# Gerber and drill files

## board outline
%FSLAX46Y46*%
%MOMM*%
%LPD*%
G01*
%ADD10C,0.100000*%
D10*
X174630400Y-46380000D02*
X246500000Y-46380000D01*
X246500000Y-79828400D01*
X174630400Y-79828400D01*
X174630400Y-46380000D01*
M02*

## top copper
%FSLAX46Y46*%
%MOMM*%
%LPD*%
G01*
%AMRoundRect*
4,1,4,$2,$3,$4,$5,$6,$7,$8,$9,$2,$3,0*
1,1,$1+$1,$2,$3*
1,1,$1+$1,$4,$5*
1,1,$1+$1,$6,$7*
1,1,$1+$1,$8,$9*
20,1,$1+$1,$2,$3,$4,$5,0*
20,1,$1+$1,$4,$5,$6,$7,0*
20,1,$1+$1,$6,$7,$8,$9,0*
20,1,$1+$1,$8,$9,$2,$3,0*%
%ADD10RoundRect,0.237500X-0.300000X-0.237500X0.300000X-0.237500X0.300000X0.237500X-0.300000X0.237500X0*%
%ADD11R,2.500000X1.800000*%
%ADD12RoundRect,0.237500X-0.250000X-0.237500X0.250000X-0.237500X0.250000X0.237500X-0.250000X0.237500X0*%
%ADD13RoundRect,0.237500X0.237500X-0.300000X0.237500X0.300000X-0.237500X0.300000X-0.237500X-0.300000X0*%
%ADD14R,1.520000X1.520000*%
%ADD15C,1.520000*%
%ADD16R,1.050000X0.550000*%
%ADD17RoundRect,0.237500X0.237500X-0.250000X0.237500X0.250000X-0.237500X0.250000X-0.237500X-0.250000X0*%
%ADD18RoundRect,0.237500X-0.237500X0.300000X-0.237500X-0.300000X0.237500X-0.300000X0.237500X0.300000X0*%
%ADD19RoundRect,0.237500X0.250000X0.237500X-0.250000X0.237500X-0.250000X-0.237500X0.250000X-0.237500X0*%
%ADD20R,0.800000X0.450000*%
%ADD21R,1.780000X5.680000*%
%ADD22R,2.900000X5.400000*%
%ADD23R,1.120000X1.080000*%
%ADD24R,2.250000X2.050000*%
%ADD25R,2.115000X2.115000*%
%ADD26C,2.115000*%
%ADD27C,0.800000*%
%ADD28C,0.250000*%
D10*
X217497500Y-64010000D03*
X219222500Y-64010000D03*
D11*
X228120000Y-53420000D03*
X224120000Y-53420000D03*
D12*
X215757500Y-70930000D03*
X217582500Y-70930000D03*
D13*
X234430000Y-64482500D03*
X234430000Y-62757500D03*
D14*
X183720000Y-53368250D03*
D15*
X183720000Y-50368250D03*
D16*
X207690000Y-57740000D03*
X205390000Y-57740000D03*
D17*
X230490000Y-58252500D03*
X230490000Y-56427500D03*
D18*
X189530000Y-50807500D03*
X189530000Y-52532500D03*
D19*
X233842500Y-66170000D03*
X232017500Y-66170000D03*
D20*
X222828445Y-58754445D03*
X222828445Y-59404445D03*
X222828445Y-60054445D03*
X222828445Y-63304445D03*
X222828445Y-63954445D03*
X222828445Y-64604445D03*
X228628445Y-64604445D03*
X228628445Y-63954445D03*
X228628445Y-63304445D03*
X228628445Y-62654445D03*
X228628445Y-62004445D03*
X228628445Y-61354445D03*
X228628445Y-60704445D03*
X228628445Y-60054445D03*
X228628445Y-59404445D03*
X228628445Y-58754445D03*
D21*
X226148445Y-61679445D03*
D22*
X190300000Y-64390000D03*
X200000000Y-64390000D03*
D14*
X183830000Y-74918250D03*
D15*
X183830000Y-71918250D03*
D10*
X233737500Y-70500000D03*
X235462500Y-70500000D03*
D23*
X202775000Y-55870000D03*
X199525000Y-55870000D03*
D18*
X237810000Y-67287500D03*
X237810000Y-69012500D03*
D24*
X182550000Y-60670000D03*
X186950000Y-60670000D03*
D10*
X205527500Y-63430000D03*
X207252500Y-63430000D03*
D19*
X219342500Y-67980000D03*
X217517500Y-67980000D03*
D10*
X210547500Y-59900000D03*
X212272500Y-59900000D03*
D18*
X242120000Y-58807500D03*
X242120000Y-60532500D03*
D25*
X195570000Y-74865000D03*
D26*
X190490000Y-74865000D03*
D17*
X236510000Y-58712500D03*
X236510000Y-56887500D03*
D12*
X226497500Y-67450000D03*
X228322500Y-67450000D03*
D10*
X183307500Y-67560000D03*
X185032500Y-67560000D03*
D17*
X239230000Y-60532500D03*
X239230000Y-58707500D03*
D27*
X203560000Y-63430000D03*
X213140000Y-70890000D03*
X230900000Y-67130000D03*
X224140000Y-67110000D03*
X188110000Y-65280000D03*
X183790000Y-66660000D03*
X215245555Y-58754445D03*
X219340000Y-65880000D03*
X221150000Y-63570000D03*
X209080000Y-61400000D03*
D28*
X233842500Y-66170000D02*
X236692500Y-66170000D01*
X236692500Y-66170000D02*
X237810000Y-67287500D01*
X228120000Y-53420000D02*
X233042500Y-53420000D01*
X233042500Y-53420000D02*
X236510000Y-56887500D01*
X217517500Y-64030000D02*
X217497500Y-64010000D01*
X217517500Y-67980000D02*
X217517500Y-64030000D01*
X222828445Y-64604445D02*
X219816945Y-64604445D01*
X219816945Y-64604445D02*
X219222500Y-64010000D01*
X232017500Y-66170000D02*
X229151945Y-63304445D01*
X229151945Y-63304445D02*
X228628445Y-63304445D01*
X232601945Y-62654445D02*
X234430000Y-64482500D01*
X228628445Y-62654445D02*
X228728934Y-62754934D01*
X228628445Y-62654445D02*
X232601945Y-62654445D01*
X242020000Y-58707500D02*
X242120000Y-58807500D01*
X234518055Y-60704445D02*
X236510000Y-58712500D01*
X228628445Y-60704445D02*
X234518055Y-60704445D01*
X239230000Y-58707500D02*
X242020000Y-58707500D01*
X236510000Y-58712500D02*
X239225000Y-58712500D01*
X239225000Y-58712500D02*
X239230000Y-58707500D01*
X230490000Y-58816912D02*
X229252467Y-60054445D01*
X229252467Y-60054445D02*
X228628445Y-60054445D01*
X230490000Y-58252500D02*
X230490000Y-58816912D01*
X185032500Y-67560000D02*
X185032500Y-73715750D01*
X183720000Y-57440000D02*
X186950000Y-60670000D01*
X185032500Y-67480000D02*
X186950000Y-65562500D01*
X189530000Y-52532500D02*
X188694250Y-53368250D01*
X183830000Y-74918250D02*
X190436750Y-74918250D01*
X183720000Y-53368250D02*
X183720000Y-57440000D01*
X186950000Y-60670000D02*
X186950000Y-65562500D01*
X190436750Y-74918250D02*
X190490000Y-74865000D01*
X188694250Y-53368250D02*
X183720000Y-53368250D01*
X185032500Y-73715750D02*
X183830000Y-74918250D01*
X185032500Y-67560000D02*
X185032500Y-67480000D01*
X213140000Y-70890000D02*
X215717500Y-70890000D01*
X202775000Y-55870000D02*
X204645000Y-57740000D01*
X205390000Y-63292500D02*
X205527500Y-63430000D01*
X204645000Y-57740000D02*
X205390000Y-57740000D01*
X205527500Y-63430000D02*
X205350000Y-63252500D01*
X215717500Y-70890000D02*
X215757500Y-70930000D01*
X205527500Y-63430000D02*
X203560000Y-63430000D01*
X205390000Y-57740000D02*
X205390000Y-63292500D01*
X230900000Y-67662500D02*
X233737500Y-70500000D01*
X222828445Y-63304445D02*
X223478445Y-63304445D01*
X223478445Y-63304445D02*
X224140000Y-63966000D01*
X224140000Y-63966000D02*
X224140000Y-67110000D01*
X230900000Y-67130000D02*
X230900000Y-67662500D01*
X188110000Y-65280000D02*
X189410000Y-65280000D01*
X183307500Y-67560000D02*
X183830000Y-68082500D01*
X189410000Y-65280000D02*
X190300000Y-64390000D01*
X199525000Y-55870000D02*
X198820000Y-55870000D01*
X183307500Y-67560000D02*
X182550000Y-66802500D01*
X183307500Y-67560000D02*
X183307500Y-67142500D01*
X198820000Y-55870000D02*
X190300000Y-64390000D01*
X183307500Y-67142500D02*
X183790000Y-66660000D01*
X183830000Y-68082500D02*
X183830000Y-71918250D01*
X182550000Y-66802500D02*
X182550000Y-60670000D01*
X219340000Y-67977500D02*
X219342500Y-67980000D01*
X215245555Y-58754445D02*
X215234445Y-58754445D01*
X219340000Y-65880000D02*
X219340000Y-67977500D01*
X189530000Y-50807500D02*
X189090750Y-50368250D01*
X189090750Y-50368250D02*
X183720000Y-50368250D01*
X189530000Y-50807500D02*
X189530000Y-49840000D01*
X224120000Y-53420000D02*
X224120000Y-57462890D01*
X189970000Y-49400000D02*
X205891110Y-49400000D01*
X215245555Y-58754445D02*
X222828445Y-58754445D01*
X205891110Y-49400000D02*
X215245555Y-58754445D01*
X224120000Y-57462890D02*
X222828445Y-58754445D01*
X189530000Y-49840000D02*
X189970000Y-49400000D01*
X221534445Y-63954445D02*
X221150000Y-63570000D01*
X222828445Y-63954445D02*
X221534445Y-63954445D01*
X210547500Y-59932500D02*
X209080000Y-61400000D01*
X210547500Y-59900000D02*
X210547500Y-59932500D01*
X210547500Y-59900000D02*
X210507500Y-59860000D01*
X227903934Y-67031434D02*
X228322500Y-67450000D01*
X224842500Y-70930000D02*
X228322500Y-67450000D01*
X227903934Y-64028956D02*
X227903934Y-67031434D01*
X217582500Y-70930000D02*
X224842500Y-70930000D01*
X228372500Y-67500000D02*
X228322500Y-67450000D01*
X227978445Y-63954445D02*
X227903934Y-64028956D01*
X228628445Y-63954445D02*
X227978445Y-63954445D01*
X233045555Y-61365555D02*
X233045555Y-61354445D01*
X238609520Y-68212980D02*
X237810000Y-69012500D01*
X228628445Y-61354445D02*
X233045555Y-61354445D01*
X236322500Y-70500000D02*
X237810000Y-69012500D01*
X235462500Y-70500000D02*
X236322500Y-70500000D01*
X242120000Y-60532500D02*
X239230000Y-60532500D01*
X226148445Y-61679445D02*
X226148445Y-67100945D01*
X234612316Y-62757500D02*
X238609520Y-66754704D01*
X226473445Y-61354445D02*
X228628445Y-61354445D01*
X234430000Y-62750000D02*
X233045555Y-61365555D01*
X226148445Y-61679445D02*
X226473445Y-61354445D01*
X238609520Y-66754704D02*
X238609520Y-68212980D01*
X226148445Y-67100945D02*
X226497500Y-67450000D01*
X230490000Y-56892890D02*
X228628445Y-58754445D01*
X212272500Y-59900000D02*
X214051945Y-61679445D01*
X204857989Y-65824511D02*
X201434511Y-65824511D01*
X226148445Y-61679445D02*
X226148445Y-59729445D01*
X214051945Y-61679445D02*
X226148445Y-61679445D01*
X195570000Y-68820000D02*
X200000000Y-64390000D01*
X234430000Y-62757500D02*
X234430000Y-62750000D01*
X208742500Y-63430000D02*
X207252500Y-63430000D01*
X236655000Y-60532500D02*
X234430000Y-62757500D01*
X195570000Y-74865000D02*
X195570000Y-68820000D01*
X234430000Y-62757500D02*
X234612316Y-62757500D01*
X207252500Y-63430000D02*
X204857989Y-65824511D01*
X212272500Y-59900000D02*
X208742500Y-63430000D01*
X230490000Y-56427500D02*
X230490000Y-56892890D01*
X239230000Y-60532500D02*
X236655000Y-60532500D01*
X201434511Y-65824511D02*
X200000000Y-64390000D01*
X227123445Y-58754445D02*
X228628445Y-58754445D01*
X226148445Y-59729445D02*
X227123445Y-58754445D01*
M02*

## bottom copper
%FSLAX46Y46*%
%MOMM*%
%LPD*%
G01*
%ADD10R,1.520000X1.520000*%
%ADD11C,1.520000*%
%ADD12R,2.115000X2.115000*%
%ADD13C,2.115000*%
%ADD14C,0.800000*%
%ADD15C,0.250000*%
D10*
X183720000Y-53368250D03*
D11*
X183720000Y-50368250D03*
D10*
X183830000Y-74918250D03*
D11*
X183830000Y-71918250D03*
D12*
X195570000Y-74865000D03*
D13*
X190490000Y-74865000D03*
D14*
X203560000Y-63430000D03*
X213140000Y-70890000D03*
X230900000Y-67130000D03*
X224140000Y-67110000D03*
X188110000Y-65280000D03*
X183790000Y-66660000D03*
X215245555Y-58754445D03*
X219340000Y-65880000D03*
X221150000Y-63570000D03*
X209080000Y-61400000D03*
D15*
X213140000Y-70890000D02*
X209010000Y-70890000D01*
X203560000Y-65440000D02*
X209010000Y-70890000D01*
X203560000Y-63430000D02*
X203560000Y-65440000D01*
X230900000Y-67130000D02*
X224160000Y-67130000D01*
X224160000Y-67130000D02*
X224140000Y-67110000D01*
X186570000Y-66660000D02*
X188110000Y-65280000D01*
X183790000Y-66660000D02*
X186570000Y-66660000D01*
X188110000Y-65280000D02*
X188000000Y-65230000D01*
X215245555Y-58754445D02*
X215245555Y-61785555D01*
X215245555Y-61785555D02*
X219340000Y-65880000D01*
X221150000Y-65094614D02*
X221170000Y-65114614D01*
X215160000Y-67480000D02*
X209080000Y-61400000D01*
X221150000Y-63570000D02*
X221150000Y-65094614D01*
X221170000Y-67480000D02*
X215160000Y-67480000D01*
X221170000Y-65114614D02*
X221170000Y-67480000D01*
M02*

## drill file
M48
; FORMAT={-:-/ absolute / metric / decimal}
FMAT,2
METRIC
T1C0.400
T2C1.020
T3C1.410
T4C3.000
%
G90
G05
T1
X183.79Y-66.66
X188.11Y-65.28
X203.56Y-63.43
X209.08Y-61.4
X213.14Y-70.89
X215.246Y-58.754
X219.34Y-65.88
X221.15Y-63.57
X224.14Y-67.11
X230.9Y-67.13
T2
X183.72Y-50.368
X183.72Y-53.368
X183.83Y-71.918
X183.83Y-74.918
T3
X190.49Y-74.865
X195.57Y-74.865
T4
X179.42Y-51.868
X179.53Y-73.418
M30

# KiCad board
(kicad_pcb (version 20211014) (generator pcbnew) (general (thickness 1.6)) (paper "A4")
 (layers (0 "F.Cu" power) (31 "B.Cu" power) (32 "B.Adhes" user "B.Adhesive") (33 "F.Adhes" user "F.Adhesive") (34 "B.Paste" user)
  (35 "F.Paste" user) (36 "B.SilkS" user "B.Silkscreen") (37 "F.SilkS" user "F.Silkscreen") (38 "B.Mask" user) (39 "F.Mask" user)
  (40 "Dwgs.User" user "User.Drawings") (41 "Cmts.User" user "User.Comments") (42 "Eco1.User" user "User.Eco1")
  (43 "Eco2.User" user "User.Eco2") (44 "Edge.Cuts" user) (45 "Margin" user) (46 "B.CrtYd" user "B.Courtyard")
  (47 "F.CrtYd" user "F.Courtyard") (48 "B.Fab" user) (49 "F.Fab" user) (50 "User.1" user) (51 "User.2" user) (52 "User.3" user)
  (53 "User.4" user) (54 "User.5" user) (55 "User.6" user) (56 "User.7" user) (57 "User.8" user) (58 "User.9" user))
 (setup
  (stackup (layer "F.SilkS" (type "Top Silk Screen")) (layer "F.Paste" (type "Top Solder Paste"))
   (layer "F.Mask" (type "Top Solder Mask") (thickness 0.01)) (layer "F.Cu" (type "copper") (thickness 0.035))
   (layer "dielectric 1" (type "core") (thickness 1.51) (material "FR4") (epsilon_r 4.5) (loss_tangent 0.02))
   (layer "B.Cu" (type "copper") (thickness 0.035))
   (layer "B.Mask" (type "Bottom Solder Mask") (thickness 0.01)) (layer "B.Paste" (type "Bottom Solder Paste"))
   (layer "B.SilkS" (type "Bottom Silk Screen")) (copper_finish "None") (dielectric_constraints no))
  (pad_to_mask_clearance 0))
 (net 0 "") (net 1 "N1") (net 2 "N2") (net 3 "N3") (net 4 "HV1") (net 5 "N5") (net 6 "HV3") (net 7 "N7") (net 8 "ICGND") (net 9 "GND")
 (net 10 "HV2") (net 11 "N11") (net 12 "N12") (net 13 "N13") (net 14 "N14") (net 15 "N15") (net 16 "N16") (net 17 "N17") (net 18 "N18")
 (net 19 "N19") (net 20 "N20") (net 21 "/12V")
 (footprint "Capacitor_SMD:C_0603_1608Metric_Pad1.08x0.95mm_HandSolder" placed (layer "F.Cu") (at 218.36 64.01)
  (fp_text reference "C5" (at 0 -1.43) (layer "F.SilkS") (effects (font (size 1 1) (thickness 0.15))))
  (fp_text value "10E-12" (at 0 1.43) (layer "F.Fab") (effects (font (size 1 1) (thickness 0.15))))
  (pad "1" smd roundrect locked (at -0.8625 0) (size 1.075 0.95) (layers "F.Cu" "F.Paste" "F.Mask") (roundrect_rratio 0.25) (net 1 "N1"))
  (pad "2" smd roundrect locked (at 0.8625 0) (size 1.075 0.95) (layers "F.Cu" "F.Paste" "F.Mask") (roundrect_rratio 0.25) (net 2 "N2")))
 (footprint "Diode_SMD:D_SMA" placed (layer "F.Cu") (at 226.12 53.42 180)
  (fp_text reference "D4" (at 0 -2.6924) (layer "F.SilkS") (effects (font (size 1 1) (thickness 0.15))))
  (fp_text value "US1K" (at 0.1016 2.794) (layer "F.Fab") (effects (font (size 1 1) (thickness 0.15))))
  (pad "1" smd rect locked (at -2 0 180) (size 2.5 1.8) (layers "F.Cu" "F.Paste" "F.Mask") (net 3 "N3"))
  (pad "2" smd rect locked (at 2 0 180) (size 2.5 1.8) (layers "F.Cu" "F.Paste" "F.Mask") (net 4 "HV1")))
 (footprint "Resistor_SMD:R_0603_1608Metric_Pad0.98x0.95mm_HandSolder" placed (layer "F.Cu") (at 216.67 70.93)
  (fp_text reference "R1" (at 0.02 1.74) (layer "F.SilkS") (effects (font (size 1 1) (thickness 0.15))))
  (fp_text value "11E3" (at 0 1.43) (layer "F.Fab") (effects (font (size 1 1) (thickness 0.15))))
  (pad "1" smd roundrect locked (at -0.9125 0) (size 0.975 0.95) (layers "F.Cu" "F.Paste" "F.Mask") (roundrect_rratio 0.25) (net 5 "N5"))
  (pad "2" smd roundrect locked (at 0.9125 0) (size 0.975 0.95) (layers "F.Cu" "F.Paste" "F.Mask") (roundrect_rratio 0.25) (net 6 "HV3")))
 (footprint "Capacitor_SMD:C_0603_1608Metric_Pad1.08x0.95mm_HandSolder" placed (layer "F.Cu") (at 234.43 63.62 90)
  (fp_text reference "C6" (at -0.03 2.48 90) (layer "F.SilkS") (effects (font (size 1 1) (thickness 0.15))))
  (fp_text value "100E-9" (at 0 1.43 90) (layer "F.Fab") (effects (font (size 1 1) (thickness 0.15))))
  (pad "1" smd roundrect locked (at -0.8625 0 90) (size 1.075 0.95) (layers "F.Cu" "F.Paste" "F.Mask") (roundrect_rratio 0.25) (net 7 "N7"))
  (pad "2" smd roundrect locked (at 0.8625 0 90) (size 1.075 0.95) (layers "F.Cu" "F.Paste" "F.Mask") (roundrect_rratio 0.25)
   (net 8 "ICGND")))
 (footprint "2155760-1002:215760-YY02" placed (layer "F.Cu") (at 183.72 53.36825 -90)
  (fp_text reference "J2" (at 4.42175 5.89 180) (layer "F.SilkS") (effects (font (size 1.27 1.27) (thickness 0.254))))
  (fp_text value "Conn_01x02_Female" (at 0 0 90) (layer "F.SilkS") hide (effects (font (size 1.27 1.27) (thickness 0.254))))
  (pad "" np_thru_hole circle locked (at -1.5 4.3 270) (size 3 3) (drill 3) (layers *.Cu *.Mask))
  (pad "1" thru_hole rect locked (at 0 0 270) (size 1.52 1.52) (drill 1.02) (layers *.Cu *.Mask) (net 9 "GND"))
  (pad "2" thru_hole circle locked (at -3 0 270) (size 1.52 1.52) (drill 1.02) (layers *.Cu *.Mask) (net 4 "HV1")))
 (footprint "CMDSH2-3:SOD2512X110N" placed (layer "F.Cu") (at 206.54 57.74 180)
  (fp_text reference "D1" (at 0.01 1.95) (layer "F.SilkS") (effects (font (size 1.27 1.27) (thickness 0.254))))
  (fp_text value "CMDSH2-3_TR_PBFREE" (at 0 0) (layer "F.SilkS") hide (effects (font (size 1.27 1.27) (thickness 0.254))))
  (pad "1" smd rect locked (at -1.15 0 270) (size 0.55 1.05) (layers "F.Cu" "F.Paste" "F.Mask") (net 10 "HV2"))
  (pad "2" smd rect locked (at 1.15 0 270) (size 0.55 1.05) (layers "F.Cu" "F.Paste" "F.Mask") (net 5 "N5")))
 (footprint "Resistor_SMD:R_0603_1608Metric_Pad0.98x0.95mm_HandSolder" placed (layer "F.Cu") (at 230.49 57.34 90)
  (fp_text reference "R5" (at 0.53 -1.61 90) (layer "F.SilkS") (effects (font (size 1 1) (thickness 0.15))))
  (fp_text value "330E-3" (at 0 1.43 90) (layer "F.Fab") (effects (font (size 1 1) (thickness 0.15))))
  (pad "1" smd roundrect locked (at -0.9125 0 90) (size 0.975 0.95) (layers "F.Cu" "F.Paste" "F.Mask") (roundrect_rratio 0.25)
   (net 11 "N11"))
  (pad "2" smd roundrect locked (at 0.9125 0 90) (size 0.975 0.95) (layers "F.Cu" "F.Paste" "F.Mask") (roundrect_rratio 0.25)
   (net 8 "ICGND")))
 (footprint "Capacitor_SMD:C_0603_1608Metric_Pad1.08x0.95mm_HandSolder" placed (layer "F.Cu") (at 189.53 51.67 -90)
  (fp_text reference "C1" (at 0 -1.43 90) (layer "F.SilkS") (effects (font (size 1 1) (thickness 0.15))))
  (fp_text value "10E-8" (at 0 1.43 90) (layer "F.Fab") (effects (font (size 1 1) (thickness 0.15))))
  (pad "1" smd roundrect locked (at -0.8625 0 270) (size 1.075 0.95) (layers "F.Cu" "F.Paste" "F.Mask") (roundrect_rratio 0.25)
   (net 4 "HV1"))
  (pad "2" smd roundrect locked (at 0.8625 0 270) (size 1.075 0.95) (layers "F.Cu" "F.Paste" "F.Mask") (roundrect_rratio 0.25) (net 9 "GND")))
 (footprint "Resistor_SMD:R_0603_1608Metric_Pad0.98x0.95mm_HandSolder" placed (layer "F.Cu") (at 232.93 66.17 180)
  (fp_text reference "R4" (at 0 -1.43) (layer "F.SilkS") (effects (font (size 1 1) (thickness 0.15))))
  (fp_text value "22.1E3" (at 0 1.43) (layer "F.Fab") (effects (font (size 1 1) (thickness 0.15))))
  (pad "1" smd roundrect locked (at -0.9125 0 180) (size 0.975 0.95) (layers "F.Cu" "F.Paste" "F.Mask") (roundrect_rratio 0.25)
   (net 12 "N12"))
  (pad "2" smd roundrect locked (at 0.9125 0 180) (size 0.975 0.95) (layers "F.Cu" "F.Paste" "F.Mask") (roundrect_rratio 0.25)
   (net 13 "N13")))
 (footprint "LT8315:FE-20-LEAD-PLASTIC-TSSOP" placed (layer "F.Cu") (at 225.728445 61.679445 -90)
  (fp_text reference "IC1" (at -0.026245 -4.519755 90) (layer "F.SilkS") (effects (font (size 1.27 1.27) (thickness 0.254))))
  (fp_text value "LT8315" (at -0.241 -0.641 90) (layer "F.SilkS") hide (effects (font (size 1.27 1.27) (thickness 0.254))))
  (pad "1" smd rect (at -2.925 2.9 270) (size 0.45 0.8) (layers "F.Cu" "F.Paste" "F.Mask") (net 4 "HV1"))
  (pad "2" smd rect (at -2.275 2.9 270) (size 0.45 0.8) (layers "F.Cu" "F.Paste" "F.Mask") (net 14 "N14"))
  (pad "3" smd rect (at -1.625 2.9 270) (size 0.45 0.8) (layers "F.Cu" "F.Paste" "F.Mask") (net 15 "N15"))
  (pad "8" smd rect (at 1.625 2.9 270) (size 0.45 0.8) (layers "F.Cu" "F.Paste" "F.Mask") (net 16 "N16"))
  (pad "9" smd rect (at 2.275 2.9 270) (size 0.45 0.8) (layers "F.Cu" "F.Paste" "F.Mask") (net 10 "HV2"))
  (pad "10" smd rect (at 2.925 2.9 270) (size 0.45 0.8) (layers "F.Cu" "F.Paste" "F.Mask") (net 2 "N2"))
  (pad "11" smd rect (at 2.925 -2.9 270) (size 0.45 0.8) (layers "F.Cu" "F.Paste" "F.Mask") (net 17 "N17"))
  (pad "12" smd rect (at 2.275 -2.9 270) (size 0.45 0.8) (layers "F.Cu" "F.Paste" "F.Mask") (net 6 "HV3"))
  (pad "13" smd rect (at 1.625 -2.9 270) (size 0.45 0.8) (layers "F.Cu" "F.Paste" "F.Mask") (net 13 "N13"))
  (pad "14" smd rect (at 0.975 -2.9 270) (size 0.45 0.8) (layers "F.Cu" "F.Paste" "F.Mask") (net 7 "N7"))
  (pad "15" smd rect (at 0.325 -2.9 270) (size 0.45 0.8) (layers "F.Cu" "F.Paste" "F.Mask") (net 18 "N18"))
  (pad "16" smd rect (at -0.325 -2.9 270) (size 0.45 0.8) (layers "F.Cu" "F.Paste" "F.Mask") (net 8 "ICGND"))
  (pad "17" smd rect (at -0.975 -2.9 270) (size 0.45 0.8) (layers "F.Cu" "F.Paste" "F.Mask") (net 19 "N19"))
  (pad "18" smd rect (at -1.625 -2.9 270) (size 0.45 0.8) (layers "F.Cu" "F.Paste" "F.Mask") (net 11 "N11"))
  (pad "19" smd rect (at -2.275 -2.9 270) (size 0.45 0.8) (layers "F.Cu" "F.Paste" "F.Mask") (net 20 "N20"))
  (pad "20" smd rect (at -2.925 -2.9 270) (size 0.45 0.8) (layers "F.Cu" "F.Paste" "F.Mask") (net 8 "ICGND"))
  (pad "21" smd rect (at 0 -0.42) (size 1.78 5.68) (layers "F.Cu" "F.Paste" "F.Mask") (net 8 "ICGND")))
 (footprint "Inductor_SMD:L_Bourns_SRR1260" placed (layer "F.Cu") (at 195.15 64.39)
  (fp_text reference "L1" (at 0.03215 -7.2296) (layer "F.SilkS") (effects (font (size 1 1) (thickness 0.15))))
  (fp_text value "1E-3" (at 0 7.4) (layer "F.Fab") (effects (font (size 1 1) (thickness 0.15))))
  (pad "1" smd rect locked (at -4.85 0) (size 2.9 5.4) (layers "F.Cu" "F.Paste" "F.Mask") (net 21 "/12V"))
  (pad "2" smd rect locked (at 4.85 0) (size 2.9 5.4) (layers "F.Cu" "F.Paste" "F.Mask") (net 8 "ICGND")))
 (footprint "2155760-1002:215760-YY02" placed (layer "F.Cu") (at 183.83 74.91825 -90)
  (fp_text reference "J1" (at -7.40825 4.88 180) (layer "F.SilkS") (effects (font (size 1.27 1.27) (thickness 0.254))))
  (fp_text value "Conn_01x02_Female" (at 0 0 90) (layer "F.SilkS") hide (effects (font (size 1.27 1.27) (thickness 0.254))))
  (pad "" np_thru_hole circle locked (at -1.5 4.3 270) (size 3 3) (drill 3) (layers *.Cu *.Mask))
  (pad "1" thru_hole rect locked (at 0 0 270) (size 1.52 1.52) (drill 1.02) (layers *.Cu *.Mask) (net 9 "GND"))
  (pad "2" thru_hole circle locked (at -3 0 270) (size 1.52 1.52) (drill 1.02) (layers *.Cu *.Mask) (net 21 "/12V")))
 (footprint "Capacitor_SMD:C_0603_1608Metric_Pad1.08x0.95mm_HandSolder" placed (layer "F.Cu") (at 234.6 70.5)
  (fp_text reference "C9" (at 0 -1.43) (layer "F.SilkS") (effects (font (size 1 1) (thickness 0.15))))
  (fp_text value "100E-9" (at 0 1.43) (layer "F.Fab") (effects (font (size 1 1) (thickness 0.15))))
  (pad "1" smd roundrect locked (at -0.8625 0) (size 1.075 0.95) (layers "F.Cu" "F.Paste" "F.Mask") (roundrect_rratio 0.25) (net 16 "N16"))
  (pad "2" smd roundrect locked (at 0.8625 0) (size 1.075 0.95) (layers "F.Cu" "F.Paste" "F.Mask") (roundrect_rratio 0.25) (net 8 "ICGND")))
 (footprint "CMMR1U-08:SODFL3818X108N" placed (layer "F.Cu") (at 201.15 55.87 180)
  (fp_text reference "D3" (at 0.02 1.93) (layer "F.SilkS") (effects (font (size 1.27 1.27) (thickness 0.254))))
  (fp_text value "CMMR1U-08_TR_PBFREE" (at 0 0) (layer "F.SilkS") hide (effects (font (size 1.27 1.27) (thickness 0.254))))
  (pad "1" smd rect locked (at -1.625 0 270) (size 1.08 1.12) (layers "F.Cu" "F.Paste" "F.Mask") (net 5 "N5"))
  (pad "2" smd rect locked (at 1.625 0 270) (size 1.08 1.12) (layers "F.Cu" "F.Paste" "F.Mask") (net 21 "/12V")))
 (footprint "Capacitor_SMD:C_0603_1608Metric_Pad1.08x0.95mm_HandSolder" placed (layer "F.Cu") (at 237.81 68.15 -90)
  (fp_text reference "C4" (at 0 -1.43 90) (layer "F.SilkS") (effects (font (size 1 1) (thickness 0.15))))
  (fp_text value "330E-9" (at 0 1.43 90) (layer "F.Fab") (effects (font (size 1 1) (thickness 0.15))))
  (pad "1" smd roundrect locked (at -0.8625 0 270) (size 1.075 0.95) (layers "F.Cu" "F.Paste" "F.Mask") (roundrect_rratio 0.25)
   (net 12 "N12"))
  (pad "2" smd roundrect locked (at 0.8625 0 270) (size 1.075 0.95) (layers "F.Cu" "F.Paste" "F.Mask") (roundrect_rratio 0.25)
   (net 8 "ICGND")))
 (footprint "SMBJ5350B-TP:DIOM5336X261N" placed (layer "F.Cu") (at 184.75 60.67)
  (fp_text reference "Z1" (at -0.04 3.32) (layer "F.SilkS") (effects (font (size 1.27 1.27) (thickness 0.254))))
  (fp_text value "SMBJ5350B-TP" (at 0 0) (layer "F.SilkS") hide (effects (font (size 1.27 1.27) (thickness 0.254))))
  (pad "1" smd rect (at -2.2 0 90) (size 2.05 2.25) (layers "F.Cu" "F.Paste" "F.Mask") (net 21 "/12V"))
  (pad "2" smd rect (at 2.2 0 90) (size 2.05 2.25) (layers "F.Cu" "F.Paste" "F.Mask") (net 9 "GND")))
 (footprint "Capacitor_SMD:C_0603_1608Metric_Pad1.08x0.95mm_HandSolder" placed (layer "F.Cu") (at 206.39 63.43)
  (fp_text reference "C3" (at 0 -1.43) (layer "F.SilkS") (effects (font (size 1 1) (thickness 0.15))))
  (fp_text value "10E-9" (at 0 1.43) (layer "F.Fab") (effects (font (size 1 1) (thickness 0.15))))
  (pad "1" smd roundrect locked (at -0.8625 0) (size 1.075 0.95) (layers "F.Cu" "F.Paste" "F.Mask") (roundrect_rratio 0.25) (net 5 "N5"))
  (pad "2" smd roundrect locked (at 0.8625 0) (size 1.075 0.95) (layers "F.Cu" "F.Paste" "F.Mask") (roundrect_rratio 0.25) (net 8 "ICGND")))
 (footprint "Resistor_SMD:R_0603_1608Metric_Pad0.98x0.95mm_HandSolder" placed (layer "F.Cu") (at 218.43 67.98 180)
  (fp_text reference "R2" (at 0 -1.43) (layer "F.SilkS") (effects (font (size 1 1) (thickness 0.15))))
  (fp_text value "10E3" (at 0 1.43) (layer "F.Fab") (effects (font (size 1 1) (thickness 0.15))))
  (pad "1" smd roundrect locked (at -0.9125 0 180) (size 0.975 0.95) (layers "F.Cu" "F.Paste" "F.Mask") (roundrect_rratio 0.25)
   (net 4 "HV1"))
  (pad "2" smd roundrect locked (at 0.9125 0 180) (size 0.975 0.95) (layers "F.Cu" "F.Paste" "F.Mask") (roundrect_rratio 0.25) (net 1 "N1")))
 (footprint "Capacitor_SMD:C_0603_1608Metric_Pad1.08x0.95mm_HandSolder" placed (layer "F.Cu") (at 211.41 59.9)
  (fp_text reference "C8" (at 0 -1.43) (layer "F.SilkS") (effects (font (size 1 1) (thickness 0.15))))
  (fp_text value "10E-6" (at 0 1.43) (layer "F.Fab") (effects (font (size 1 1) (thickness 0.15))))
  (pad "1" smd roundrect locked (at -0.8625 0) (size 1.075 0.95) (layers "F.Cu" "F.Paste" "F.Mask") (roundrect_rratio 0.25) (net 10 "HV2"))
  (pad "2" smd roundrect locked (at 0.8625 0) (size 1.075 0.95) (layers "F.Cu" "F.Paste" "F.Mask") (roundrect_rratio 0.25) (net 8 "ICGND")))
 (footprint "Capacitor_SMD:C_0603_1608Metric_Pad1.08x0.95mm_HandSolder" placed (layer "F.Cu") (at 242.12 59.67 -90)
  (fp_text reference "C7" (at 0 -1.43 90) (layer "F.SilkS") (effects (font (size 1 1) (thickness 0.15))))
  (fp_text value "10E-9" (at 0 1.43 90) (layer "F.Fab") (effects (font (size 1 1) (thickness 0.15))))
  (pad "1" smd roundrect locked (at -0.8625 0 270) (size 1.075 0.95) (layers "F.Cu" "F.Paste" "F.Mask") (roundrect_rratio 0.25)
   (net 19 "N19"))
  (pad "2" smd roundrect locked (at 0.8625 0 270) (size 1.075 0.95) (layers "F.Cu" "F.Paste" "F.Mask") (roundrect_rratio 0.25)
   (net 8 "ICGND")))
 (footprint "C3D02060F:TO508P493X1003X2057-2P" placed (layer "F.Cu") (at 195.57 74.865 180)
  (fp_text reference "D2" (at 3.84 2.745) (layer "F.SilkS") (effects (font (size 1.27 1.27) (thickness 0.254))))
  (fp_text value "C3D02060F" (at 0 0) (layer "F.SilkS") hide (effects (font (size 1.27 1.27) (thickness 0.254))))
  (pad "1" thru_hole rect (at 0 0 180) (size 2.115 2.115) (drill 1.41) (layers *.Cu *.Mask) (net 8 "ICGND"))
  (pad "2" thru_hole circle (at 5.08 0 180) (size 2.115 2.115) (drill 1.41) (layers *.Cu *.Mask) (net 9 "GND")))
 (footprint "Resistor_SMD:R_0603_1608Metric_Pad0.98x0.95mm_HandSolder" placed (layer "F.Cu") (at 236.51 57.8 90)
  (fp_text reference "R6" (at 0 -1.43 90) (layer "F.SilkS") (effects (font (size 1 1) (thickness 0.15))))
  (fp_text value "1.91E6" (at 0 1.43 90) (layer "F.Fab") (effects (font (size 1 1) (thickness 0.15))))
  (pad "1" smd roundrect locked (at -0.9125 0 90) (size 0.975 0.95) (layers "F.Cu" "F.Paste" "F.Mask") (roundrect_rratio 0.25)
   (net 19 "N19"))
  (pad "2" smd roundrect locked (at 0.9125 0 90) (size 0.975 0.95) (layers "F.Cu" "F.Paste" "F.Mask") (roundrect_rratio 0.25) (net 3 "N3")))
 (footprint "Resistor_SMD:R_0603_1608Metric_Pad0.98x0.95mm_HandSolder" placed (layer "F.Cu") (at 227.41 67.45)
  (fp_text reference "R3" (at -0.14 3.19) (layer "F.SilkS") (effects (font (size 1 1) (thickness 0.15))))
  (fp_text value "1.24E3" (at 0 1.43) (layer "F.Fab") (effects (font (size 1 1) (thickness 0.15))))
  (pad "1" smd roundrect locked (at -0.9125 0) (size 0.975 0.95) (layers "F.Cu" "F.Paste" "F.Mask") (roundrect_rratio 0.25) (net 8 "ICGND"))
  (pad "2" smd roundrect locked (at 0.9125 0) (size 0.975 0.95) (layers "F.Cu" "F.Paste" "F.Mask") (roundrect_rratio 0.25) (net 6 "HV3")))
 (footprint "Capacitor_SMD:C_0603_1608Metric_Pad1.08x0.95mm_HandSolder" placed (layer "F.Cu") (at 184.17 67.56)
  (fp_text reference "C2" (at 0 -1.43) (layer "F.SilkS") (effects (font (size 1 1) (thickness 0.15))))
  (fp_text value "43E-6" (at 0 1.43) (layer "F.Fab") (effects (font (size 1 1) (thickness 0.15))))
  (pad "1" smd roundrect locked (at -0.8625 0) (size 1.075 0.95) (layers "F.Cu" "F.Paste" "F.Mask") (roundrect_rratio 0.25) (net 21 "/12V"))
  (pad "2" smd roundrect locked (at 0.8625 0) (size 1.075 0.95) (layers "F.Cu" "F.Paste" "F.Mask") (roundrect_rratio 0.25) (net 9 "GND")))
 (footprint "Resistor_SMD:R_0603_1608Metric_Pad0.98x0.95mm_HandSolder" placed (layer "F.Cu") (at 239.23 59.62 90)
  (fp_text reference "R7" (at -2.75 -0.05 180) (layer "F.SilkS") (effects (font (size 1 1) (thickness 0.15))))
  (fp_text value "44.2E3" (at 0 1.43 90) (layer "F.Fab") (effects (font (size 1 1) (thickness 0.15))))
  (pad "1" smd roundrect locked (at -0.9125 0 90) (size 0.975 0.95) (layers "F.Cu" "F.Paste" "F.Mask") (roundrect_rratio 0.25)
   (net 8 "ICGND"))
  (pad "2" smd roundrect locked (at 0.9125 0 90) (size 0.975 0.95) (layers "F.Cu" "F.Paste" "F.Mask") (roundrect_rratio 0.25) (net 19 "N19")))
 (gr_rect (start 174.6304 46.38) (end 246.5 79.8284) (layer "Edge.Cuts") (width 0.1) (fill none))
 (segment (start 233.8425 66.17) (end 236.6925 66.17) (width 0.25) (layer "F.Cu") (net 12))
 (segment (start 236.6925 66.17) (end 237.81 67.2875) (width 0.25) (layer "F.Cu") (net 12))
 (segment (start 228.12 53.42) (end 233.0425 53.42) (width 0.25) (layer "F.Cu") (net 3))
 (segment (start 233.0425 53.42) (end 236.51 56.8875) (width 0.25) (layer "F.Cu") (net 3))
 (segment (start 217.5175 64.03) (end 217.4975 64.01) (width 0.25) (layer "F.Cu") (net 1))
 (segment (start 217.5175 67.98) (end 217.5175 64.03) (width 0.25) (layer "F.Cu") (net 1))
 (segment (start 222.828445 64.604445) (end 219.816945 64.604445) (width 0.25) (layer "F.Cu") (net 2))
 (segment (start 219.816945 64.604445) (end 219.2225 64.01) (width 0.25) (layer "F.Cu") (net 2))
 (segment (start 232.0175 66.17) (end 229.151945 63.304445) (width 0.25) (layer "F.Cu") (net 13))
 (segment (start 229.151945 63.304445) (end 228.628445 63.304445) (width 0.25) (layer "F.Cu") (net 13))
 (segment (start 232.601945 62.654445) (end 234.43 64.4825) (width 0.25) (layer "F.Cu") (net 7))
 (segment (start 228.628445 62.654445) (end 228.728934 62.754934) (width 0.25) (layer "F.Cu") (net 7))
 (segment (start 228.628445 62.654445) (end 232.601945 62.654445) (width 0.25) (layer "F.Cu") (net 7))
 (segment (start 242.02 58.7075) (end 242.12 58.8075) (width 0.25) (layer "F.Cu") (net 19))
 (segment (start 234.518055 60.704445) (end 236.51 58.7125) (width 0.25) (layer "F.Cu") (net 19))
 (segment (start 228.628445 60.704445) (end 234.518055 60.704445) (width 0.25) (layer "F.Cu") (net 19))
 (segment (start 239.23 58.7075) (end 242.02 58.7075) (width 0.25) (layer "F.Cu") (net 19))
 (segment (start 236.51 58.7125) (end 239.225 58.7125) (width 0.25) (layer "F.Cu") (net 19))
 (segment (start 239.225 58.7125) (end 239.23 58.7075) (width 0.25) (layer "F.Cu") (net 19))
 (segment (start 230.49 58.816912) (end 229.252467 60.054445) (width 0.25) (layer "F.Cu") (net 11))
 (segment (start 229.252467 60.054445) (end 228.628445 60.054445) (width 0.25) (layer "F.Cu") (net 11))
 (segment (start 230.49 58.2525) (end 230.49 58.816912) (width 0.25) (layer "F.Cu") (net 11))
 (segment (start 185.0325 67.56) (end 185.0325 73.71575) (width 0.25) (layer "F.Cu") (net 9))
 (segment (start 183.72 57.44) (end 186.95 60.67) (width 0.25) (layer "F.Cu") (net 9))
 (segment (start 185.0325 67.48) (end 186.95 65.5625) (width 0.25) (layer "F.Cu") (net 9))
 (segment (start 189.53 52.5325) (end 188.69425 53.36825) (width 0.25) (layer "F.Cu") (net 9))
 (segment (start 183.83 74.91825) (end 190.43675 74.91825) (width 0.25) (layer "F.Cu") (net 9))
 (segment (start 183.72 53.36825) (end 183.72 57.44) (width 0.25) (layer "F.Cu") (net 9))
 (segment (start 186.95 60.67) (end 186.95 65.5625) (width 0.25) (layer "F.Cu") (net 9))
 (segment (start 190.43675 74.91825) (end 190.49 74.865) (width 0.25) (layer "F.Cu") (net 9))
 (segment (start 188.69425 53.36825) (end 183.72 53.36825) (width 0.25) (layer "F.Cu") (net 9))
 (segment (start 185.0325 73.71575) (end 183.83 74.91825) (width 0.25) (layer "F.Cu") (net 9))
 (segment (start 185.0325 67.56) (end 185.0325 67.48) (width 0.25) (layer "F.Cu") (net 9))
 (segment (start 213.14 70.89) (end 215.7175 70.89) (width 0.25) (layer "F.Cu") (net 5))
 (segment (start 202.775 55.87) (end 204.645 57.74) (width 0.25) (layer "F.Cu") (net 5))
 (segment (start 205.39 63.2925) (end 205.5275 63.43) (width 0.25) (layer "F.Cu") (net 5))
 (segment (start 204.645 57.74) (end 205.39 57.74) (width 0.25) (layer "F.Cu") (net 5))
 (segment (start 205.5275 63.43) (end 205.35 63.2525) (width 0.25) (layer "F.Cu") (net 5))
 (segment (start 215.7175 70.89) (end 215.7575 70.93) (width 0.25) (layer "F.Cu") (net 5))
 (segment (start 205.5275 63.43) (end 203.56 63.43) (width 0.25) (layer "F.Cu") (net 5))
 (segment (start 205.39 57.74) (end 205.39 63.2925) (width 0.25) (layer "F.Cu") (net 5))
 (via (at 203.56 63.43) (size 0.8) (drill 0.4) (layers "F.Cu" "B.Cu") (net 5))
 (via (at 213.14 70.89) (size 0.8) (drill 0.4) (layers "F.Cu" "B.Cu") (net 5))
 (segment (start 213.14 70.89) (end 209.01 70.89) (width 0.25) (layer "B.Cu") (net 5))
 (segment (start 203.56 65.44) (end 209.01 70.89) (width 0.25) (layer "B.Cu") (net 5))
 (segment (start 203.56 63.43) (end 203.56 65.44) (width 0.25) (layer "B.Cu") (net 5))
 (segment (start 230.9 67.6625) (end 233.7375 70.5) (width 0.25) (layer "F.Cu") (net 16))
 (segment (start 222.828445 63.304445) (end 223.478445 63.304445) (width 0.25) (layer "F.Cu") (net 16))
 (segment (start 223.478445 63.304445) (end 224.14 63.966) (width 0.25) (layer "F.Cu") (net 16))
 (segment (start 224.14 63.966) (end 224.14 67.11) (width 0.25) (layer "F.Cu") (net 16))
 (segment (start 230.9 67.13) (end 230.9 67.6625) (width 0.25) (layer "F.Cu") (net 16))
 (via (at 230.9 67.13) (size 0.8) (drill 0.4) (layers "F.Cu" "B.Cu") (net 16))
 (via (at 224.14 67.11) (size 0.8) (drill 0.4) (layers "F.Cu" "B.Cu") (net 16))
 (segment (start 230.9 67.13) (end 224.16 67.13) (width 0.25) (layer "B.Cu") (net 16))
 (segment (start 224.16 67.13) (end 224.14 67.11) (width 0.25) (layer "B.Cu") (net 16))
 (segment (start 188.11 65.28) (end 189.41 65.28) (width 0.25) (layer "F.Cu") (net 21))
 (segment (start 183.3075 67.56) (end 183.83 68.0825) (width 0.25) (layer "F.Cu") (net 21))
 (segment (start 189.41 65.28) (end 190.3 64.39) (width 0.25) (layer "F.Cu") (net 21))
 (segment (start 199.525 55.87) (end 198.82 55.87) (width 0.25) (layer "F.Cu") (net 21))
 (segment (start 183.3075 67.56) (end 182.55 66.8025) (width 0.25) (layer "F.Cu") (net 21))
 (segment (start 183.3075 67.56) (end 183.3075 67.1425) (width 0.25) (layer "F.Cu") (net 21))
 (segment (start 198.82 55.87) (end 190.3 64.39) (width 0.25) (layer "F.Cu") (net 21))
 (segment (start 183.3075 67.1425) (end 183.79 66.66) (width 0.25) (layer "F.Cu") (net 21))
 (segment (start 183.83 68.0825) (end 183.83 71.91825) (width 0.25) (layer "F.Cu") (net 21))
 (segment (start 182.55 66.8025) (end 182.55 60.67) (width 0.25) (layer "F.Cu") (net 21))
 (via (at 188.11 65.28) (size 0.8) (drill 0.4) (layers "F.Cu" "B.Cu") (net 21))
 (via (at 183.79 66.66) (size 0.8) (drill 0.4) (layers "F.Cu" "B.Cu") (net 21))
 (segment (start 186.57 66.66) (end 188.11 65.28) (width 0.25) (layer "B.Cu") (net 21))
 (segment (start 183.79 66.66) (end 186.57 66.66) (width 0.25) (layer "B.Cu") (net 21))
 (segment (start 188.11 65.28) (end 188 65.23) (width 0.25) (layer "B.Cu") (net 21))
 (segment (start 219.34 67.9775) (end 219.3425 67.98) (width 0.25) (layer "F.Cu") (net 4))
 (segment (start 215.245555 58.754445) (end 215.234445 58.754445) (width 0.25) (layer "F.Cu") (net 4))
 (segment (start 219.34 65.88) (end 219.34 67.9775) (width 0.25) (layer "F.Cu") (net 4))
 (segment (start 189.53 50.8075) (end 189.09075 50.36825) (width 0.25) (layer "F.Cu") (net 4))
 (segment (start 189.09075 50.36825) (end 183.72 50.36825) (width 0.25) (layer "F.Cu") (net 4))
 (segment (start 189.53 50.8075) (end 189.53 49.84) (width 0.25) (layer "F.Cu") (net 4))
 (segment (start 224.12 53.42) (end 224.12 57.46289) (width 0.25) (layer "F.Cu") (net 4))
 (segment (start 189.97 49.4) (end 205.89111 49.4) (width 0.25) (layer "F.Cu") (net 4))
 (segment (start 215.245555 58.754445) (end 222.828445 58.754445) (width 0.25) (layer "F.Cu") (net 4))
 (segment (start 205.89111 49.4) (end 215.245555 58.754445) (width 0.25) (layer "F.Cu") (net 4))
 (segment (start 224.12 57.46289) (end 222.828445 58.754445) (width 0.25) (layer "F.Cu") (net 4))
 (segment (start 189.53 49.84) (end 189.97 49.4) (width 0.25) (layer "F.Cu") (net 4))
 (via (at 215.245555 58.754445) (size 0.8) (drill 0.4) (layers "F.Cu" "B.Cu") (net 4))
 (via (at 219.34 65.88) (size 0.8) (drill 0.4) (layers "F.Cu" "B.Cu") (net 4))
 (segment (start 215.245555 58.754445) (end 215.245555 61.785555) (width 0.25) (layer "B.Cu") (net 4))
 (segment (start 215.245555 61.785555) (end 219.34 65.88) (width 0.25) (layer "B.Cu") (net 4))
 (segment (start 221.534445 63.954445) (end 221.15 63.57) (width 0.25) (layer "F.Cu") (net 10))
 (segment (start 222.828445 63.954445) (end 221.534445 63.954445) (width 0.25) (layer "F.Cu") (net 10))
 (segment (start 210.5475 59.9325) (end 209.08 61.4) (width 0.25) (layer "F.Cu") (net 10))
 (segment (start 210.5475 59.9) (end 210.5475 59.9325) (width 0.25) (layer "F.Cu") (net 10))
 (segment (start 210.5475 59.9) (end 210.5075 59.86) (width 0.25) (layer "F.Cu") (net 10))
 (via (at 221.15 63.57) (size 0.8) (drill 0.4) (layers "F.Cu" "B.Cu") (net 10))
 (via (at 209.08 61.4) (size 0.8) (drill 0.4) (layers "F.Cu" "B.Cu") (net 10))
 (segment (start 221.15 65.094614) (end 221.17 65.114614) (width 0.25) (layer "B.Cu") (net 10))
 (segment (start 215.16 67.48) (end 209.08 61.4) (width 0.25) (layer "B.Cu") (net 10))
 (segment (start 221.15 63.57) (end 221.15 65.094614) (width 0.25) (layer "B.Cu") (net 10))
 (segment (start 221.17 67.48) (end 215.16 67.48) (width 0.25) (layer "B.Cu") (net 10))
 (segment (start 221.17 65.114614) (end 221.17 67.48) (width 0.25) (layer "B.Cu") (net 10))
 (segment (start 227.903934 67.031434) (end 228.3225 67.45) (width 0.25) (layer "F.Cu") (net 6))
 (segment (start 224.8425 70.93) (end 228.3225 67.45) (width 0.25) (layer "F.Cu") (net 6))
 (segment (start 227.903934 64.028956) (end 227.903934 67.031434) (width 0.25) (layer "F.Cu") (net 6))
 (segment (start 217.5825 70.93) (end 224.8425 70.93) (width 0.25) (layer "F.Cu") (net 6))
 (segment (start 228.3725 67.5) (end 228.3225 67.45) (width 0.25) (layer "F.Cu") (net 6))
 (segment (start 227.978445 63.954445) (end 227.903934 64.028956) (width 0.25) (layer "F.Cu") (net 6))
 (segment (start 228.628445 63.954445) (end 227.978445 63.954445) (width 0.25) (layer "F.Cu") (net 6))
 (segment (start 233.045555 61.365555) (end 233.045555 61.354445) (width 0.25) (layer "F.Cu") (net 8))
 (segment (start 238.60952 68.21298) (end 237.81 69.0125) (width 0.25) (layer "F.Cu") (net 8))
 (segment (start 228.628445 61.354445) (end 233.045555 61.354445) (width 0.25) (layer "F.Cu") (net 8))
 (segment (start 236.3225 70.5) (end 237.81 69.0125) (width 0.25) (layer "F.Cu") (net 8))
 (segment (start 235.4625 70.5) (end 236.3225 70.5) (width 0.25) (layer "F.Cu") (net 8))
 (segment (start 242.12 60.5325) (end 239.23 60.5325) (width 0.25) (layer "F.Cu") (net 8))
 (segment (start 226.148445 61.679445) (end 226.148445 67.100945) (width 0.25) (layer "F.Cu") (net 8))
 (segment (start 234.612316 62.7575) (end 238.60952 66.754704) (width 0.25) (layer "F.Cu") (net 8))
 (segment (start 226.473445 61.354445) (end 228.628445 61.354445) (width 0.25) (layer "F.Cu") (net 8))
 (segment (start 234.43 62.75) (end 233.045555 61.365555) (width 0.25) (layer "F.Cu") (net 8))
 (segment (start 226.148445 61.679445) (end 226.473445 61.354445) (width 0.25) (layer "F.Cu") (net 8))
 (segment (start 238.60952 66.754704) (end 238.60952 68.21298) (width 0.25) (layer "F.Cu") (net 8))
 (segment (start 226.148445 67.100945) (end 226.4975 67.45) (width 0.25) (layer "F.Cu") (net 8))
 (segment (start 230.49 56.89289) (end 228.628445 58.754445) (width 0.25) (layer "F.Cu") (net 8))
 (segment (start 212.2725 59.9) (end 214.051945 61.679445) (width 0.25) (layer "F.Cu") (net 8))
 (segment (start 204.857989 65.824511) (end 201.434511 65.824511) (width 0.25) (layer "F.Cu") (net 8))
 (segment (start 226.148445 61.679445) (end 226.148445 59.729445) (width 0.25) (layer "F.Cu") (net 8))
 (segment (start 214.051945 61.679445) (end 226.148445 61.679445) (width 0.25) (layer "F.Cu") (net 8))
 (segment (start 195.57 68.82) (end 200 64.39) (width 0.25) (layer "F.Cu") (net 8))
 (segment (start 234.43 62.7575) (end 234.43 62.75) (width 0.25) (layer "F.Cu") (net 8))
 (segment (start 208.7425 63.43) (end 207.2525 63.43) (width 0.25) (layer "F.Cu") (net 8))
 (segment (start 236.655 60.5325) (end 234.43 62.7575) (width 0.25) (layer "F.Cu") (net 8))
 (segment (start 195.57 74.865) (end 195.57 68.82) (width 0.25) (layer "F.Cu") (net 8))
 (segment (start 234.43 62.7575) (end 234.612316 62.7575) (width 0.25) (layer "F.Cu") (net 8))
 (segment (start 207.2525 63.43) (end 204.857989 65.824511) (width 0.25) (layer "F.Cu") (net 8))
 (segment (start 212.2725 59.9) (end 208.7425 63.43) (width 0.25) (layer "F.Cu") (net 8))
 (segment (start 230.49 56.4275) (end 230.49 56.89289) (width 0.25) (layer "F.Cu") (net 8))
 (segment (start 239.23 60.5325) (end 236.655 60.5325) (width 0.25) (layer "F.Cu") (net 8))
 (segment (start 201.434511 65.824511) (end 200 64.39) (width 0.25) (layer "F.Cu") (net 8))
 (segment (start 227.123445 58.754445) (end 228.628445 58.754445) (width 0.25) (layer "F.Cu") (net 8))
 (segment (start 226.148445 59.729445) (end 227.123445 58.754445) (width 0.25) (layer "F.Cu") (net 8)))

